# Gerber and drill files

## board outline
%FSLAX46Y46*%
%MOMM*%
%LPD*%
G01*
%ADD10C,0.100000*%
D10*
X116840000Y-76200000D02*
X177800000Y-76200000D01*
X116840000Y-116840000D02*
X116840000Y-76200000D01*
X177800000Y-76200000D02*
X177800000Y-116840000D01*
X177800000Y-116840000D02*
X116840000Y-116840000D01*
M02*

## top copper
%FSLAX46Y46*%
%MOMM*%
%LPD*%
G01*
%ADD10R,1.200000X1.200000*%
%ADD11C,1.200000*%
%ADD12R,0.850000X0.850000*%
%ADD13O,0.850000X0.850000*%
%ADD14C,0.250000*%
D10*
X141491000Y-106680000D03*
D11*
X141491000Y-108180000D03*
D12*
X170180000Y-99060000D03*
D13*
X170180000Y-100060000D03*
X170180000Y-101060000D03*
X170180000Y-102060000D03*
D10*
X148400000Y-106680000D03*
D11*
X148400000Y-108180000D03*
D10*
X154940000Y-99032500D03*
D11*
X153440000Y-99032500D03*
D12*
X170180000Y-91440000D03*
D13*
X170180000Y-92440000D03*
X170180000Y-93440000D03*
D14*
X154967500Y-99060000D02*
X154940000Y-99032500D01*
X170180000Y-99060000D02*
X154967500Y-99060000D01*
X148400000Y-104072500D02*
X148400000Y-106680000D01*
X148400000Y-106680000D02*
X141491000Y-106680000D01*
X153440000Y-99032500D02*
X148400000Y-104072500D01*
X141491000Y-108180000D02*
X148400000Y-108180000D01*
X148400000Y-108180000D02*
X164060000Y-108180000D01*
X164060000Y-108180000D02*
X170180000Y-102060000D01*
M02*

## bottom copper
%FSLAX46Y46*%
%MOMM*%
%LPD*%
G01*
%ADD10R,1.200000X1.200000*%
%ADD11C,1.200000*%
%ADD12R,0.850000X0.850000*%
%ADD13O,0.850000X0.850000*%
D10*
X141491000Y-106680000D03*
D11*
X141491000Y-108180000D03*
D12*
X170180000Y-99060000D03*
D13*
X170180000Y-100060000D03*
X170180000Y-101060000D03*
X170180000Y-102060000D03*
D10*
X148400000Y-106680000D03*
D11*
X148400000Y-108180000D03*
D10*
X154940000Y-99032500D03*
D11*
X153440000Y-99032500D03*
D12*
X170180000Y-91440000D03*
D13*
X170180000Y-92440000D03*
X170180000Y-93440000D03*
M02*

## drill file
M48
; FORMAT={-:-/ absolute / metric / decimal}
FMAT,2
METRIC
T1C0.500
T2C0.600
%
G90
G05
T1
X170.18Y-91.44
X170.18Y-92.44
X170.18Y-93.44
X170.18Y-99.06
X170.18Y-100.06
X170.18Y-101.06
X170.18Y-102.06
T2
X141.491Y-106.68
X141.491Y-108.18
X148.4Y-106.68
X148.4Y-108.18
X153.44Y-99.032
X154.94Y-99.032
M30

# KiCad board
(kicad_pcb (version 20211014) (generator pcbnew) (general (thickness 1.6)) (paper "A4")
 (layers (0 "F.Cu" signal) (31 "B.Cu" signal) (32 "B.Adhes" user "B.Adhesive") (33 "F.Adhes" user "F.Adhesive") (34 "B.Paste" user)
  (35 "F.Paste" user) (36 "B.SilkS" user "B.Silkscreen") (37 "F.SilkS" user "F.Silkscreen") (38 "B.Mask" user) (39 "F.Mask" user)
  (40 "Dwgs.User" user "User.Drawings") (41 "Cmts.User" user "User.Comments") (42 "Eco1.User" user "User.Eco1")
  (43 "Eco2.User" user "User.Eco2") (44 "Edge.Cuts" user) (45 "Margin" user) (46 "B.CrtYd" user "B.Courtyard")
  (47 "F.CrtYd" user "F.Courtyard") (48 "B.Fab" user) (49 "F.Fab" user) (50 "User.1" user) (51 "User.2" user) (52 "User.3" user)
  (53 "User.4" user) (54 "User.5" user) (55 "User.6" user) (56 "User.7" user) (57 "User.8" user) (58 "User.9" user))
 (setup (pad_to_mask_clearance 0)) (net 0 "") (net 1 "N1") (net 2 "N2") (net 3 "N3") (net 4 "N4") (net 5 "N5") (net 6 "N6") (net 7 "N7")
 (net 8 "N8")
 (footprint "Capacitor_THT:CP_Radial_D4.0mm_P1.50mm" (layer "F.Cu") (at 141.491 106.68 -90)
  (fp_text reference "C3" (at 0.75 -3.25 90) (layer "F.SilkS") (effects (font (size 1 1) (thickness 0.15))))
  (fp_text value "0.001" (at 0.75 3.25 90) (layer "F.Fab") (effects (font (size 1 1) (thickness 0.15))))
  (pad "1" thru_hole rect (at 0 0 270) (size 1.2 1.2) (drill 0.6) (layers *.Cu *.Mask) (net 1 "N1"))
  (pad "2" thru_hole circle (at 1.5 0 270) (size 1.2 1.2) (drill 0.6) (layers *.Cu *.Mask) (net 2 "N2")))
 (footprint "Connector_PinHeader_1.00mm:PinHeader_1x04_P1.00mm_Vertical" (layer "F.Cu") (at 170.18 99.06)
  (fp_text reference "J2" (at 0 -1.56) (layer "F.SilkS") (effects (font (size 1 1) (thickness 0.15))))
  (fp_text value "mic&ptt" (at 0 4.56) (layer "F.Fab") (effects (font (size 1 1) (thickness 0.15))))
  (pad "1" thru_hole rect (at 0 0) (size 0.85 0.85) (drill 0.5) (layers *.Cu *.Mask) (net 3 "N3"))
  (pad "2" thru_hole oval (at 0 1) (size 0.85 0.85) (drill 0.5) (layers *.Cu *.Mask) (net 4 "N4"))
  (pad "3" thru_hole oval (at 0 2) (size 0.85 0.85) (drill 0.5) (layers *.Cu *.Mask) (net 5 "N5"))
  (pad "4" thru_hole oval (at 0 3) (size 0.85 0.85) (drill 0.5) (layers *.Cu *.Mask) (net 2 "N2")))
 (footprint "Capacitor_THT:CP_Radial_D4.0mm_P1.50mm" (layer "F.Cu") (at 148.4 106.68 -90)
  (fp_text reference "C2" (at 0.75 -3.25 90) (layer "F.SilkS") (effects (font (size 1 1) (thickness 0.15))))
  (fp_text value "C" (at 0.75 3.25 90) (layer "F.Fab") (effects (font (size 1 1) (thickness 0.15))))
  (pad "1" thru_hole rect (at 0 0 270) (size 1.2 1.2) (drill 0.6) (layers *.Cu *.Mask) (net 1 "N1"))
  (pad "2" thru_hole circle (at 1.5 0 270) (size 1.2 1.2) (drill 0.6) (layers *.Cu *.Mask) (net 2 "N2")))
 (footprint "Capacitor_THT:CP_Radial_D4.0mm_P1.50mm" (layer "F.Cu") (at 154.94 99.0325 180)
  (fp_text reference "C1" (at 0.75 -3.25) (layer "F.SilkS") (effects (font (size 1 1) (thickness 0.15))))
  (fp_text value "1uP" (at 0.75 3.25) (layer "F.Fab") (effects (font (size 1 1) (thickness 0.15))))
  (pad "1" thru_hole rect (at 0 0 180) (size 1.2 1.2) (drill 0.6) (layers *.Cu *.Mask) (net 3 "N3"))
  (pad "2" thru_hole circle (at 1.5 0 180) (size 1.2 1.2) (drill 0.6) (layers *.Cu *.Mask) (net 1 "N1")))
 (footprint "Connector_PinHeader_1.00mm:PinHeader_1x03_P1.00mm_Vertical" (layer "F.Cu") (at 170.18 91.44)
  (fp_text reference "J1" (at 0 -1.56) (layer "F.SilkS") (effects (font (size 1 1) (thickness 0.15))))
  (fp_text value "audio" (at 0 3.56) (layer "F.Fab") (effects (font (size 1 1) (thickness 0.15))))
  (pad "1" thru_hole rect (at 0 0) (size 0.85 0.85) (drill 0.5) (layers *.Cu *.Mask) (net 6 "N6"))
  (pad "2" thru_hole oval (at 0 1) (size 0.85 0.85) (drill 0.5) (layers *.Cu *.Mask) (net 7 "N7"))
  (pad "3" thru_hole oval (at 0 2) (size 0.85 0.85) (drill 0.5) (layers *.Cu *.Mask) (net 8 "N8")))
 (gr_line (start 116.84 76.2) (end 177.8 76.2) (layer "Edge.Cuts") (width 0.1))
 (gr_line (start 116.84 116.84) (end 116.84 76.2) (layer "Edge.Cuts") (width 0.1))
 (gr_line (start 177.8 76.2) (end 177.8 116.84) (layer "Edge.Cuts") (width 0.1))
 (gr_line (start 177.8 116.84) (end 116.84 116.84) (layer "Edge.Cuts") (width 0.1))
 (segment (start 154.9675 99.06) (end 154.94 99.0325) (width 0.25) (layer "F.Cu") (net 3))
 (segment (start 170.18 99.06) (end 154.9675 99.06) (width 0.25) (layer "F.Cu") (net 3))
 (segment (start 148.4 104.0725) (end 148.4 106.68) (width 0.25) (layer "F.Cu") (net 1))
 (segment (start 148.4 106.68) (end 141.491 106.68) (width 0.25) (layer "F.Cu") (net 1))
 (segment (start 153.44 99.0325) (end 148.4 104.0725) (width 0.25) (layer "F.Cu") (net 1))
 (segment (start 141.491 108.18) (end 148.4 108.18) (width 0.25) (layer "F.Cu") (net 2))
 (segment (start 148.4 108.18) (end 164.06 108.18) (width 0.25) (layer "F.Cu") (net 2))
 (segment (start 164.06 108.18) (end 170.18 102.06) (width 0.25) (layer "F.Cu") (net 2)))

